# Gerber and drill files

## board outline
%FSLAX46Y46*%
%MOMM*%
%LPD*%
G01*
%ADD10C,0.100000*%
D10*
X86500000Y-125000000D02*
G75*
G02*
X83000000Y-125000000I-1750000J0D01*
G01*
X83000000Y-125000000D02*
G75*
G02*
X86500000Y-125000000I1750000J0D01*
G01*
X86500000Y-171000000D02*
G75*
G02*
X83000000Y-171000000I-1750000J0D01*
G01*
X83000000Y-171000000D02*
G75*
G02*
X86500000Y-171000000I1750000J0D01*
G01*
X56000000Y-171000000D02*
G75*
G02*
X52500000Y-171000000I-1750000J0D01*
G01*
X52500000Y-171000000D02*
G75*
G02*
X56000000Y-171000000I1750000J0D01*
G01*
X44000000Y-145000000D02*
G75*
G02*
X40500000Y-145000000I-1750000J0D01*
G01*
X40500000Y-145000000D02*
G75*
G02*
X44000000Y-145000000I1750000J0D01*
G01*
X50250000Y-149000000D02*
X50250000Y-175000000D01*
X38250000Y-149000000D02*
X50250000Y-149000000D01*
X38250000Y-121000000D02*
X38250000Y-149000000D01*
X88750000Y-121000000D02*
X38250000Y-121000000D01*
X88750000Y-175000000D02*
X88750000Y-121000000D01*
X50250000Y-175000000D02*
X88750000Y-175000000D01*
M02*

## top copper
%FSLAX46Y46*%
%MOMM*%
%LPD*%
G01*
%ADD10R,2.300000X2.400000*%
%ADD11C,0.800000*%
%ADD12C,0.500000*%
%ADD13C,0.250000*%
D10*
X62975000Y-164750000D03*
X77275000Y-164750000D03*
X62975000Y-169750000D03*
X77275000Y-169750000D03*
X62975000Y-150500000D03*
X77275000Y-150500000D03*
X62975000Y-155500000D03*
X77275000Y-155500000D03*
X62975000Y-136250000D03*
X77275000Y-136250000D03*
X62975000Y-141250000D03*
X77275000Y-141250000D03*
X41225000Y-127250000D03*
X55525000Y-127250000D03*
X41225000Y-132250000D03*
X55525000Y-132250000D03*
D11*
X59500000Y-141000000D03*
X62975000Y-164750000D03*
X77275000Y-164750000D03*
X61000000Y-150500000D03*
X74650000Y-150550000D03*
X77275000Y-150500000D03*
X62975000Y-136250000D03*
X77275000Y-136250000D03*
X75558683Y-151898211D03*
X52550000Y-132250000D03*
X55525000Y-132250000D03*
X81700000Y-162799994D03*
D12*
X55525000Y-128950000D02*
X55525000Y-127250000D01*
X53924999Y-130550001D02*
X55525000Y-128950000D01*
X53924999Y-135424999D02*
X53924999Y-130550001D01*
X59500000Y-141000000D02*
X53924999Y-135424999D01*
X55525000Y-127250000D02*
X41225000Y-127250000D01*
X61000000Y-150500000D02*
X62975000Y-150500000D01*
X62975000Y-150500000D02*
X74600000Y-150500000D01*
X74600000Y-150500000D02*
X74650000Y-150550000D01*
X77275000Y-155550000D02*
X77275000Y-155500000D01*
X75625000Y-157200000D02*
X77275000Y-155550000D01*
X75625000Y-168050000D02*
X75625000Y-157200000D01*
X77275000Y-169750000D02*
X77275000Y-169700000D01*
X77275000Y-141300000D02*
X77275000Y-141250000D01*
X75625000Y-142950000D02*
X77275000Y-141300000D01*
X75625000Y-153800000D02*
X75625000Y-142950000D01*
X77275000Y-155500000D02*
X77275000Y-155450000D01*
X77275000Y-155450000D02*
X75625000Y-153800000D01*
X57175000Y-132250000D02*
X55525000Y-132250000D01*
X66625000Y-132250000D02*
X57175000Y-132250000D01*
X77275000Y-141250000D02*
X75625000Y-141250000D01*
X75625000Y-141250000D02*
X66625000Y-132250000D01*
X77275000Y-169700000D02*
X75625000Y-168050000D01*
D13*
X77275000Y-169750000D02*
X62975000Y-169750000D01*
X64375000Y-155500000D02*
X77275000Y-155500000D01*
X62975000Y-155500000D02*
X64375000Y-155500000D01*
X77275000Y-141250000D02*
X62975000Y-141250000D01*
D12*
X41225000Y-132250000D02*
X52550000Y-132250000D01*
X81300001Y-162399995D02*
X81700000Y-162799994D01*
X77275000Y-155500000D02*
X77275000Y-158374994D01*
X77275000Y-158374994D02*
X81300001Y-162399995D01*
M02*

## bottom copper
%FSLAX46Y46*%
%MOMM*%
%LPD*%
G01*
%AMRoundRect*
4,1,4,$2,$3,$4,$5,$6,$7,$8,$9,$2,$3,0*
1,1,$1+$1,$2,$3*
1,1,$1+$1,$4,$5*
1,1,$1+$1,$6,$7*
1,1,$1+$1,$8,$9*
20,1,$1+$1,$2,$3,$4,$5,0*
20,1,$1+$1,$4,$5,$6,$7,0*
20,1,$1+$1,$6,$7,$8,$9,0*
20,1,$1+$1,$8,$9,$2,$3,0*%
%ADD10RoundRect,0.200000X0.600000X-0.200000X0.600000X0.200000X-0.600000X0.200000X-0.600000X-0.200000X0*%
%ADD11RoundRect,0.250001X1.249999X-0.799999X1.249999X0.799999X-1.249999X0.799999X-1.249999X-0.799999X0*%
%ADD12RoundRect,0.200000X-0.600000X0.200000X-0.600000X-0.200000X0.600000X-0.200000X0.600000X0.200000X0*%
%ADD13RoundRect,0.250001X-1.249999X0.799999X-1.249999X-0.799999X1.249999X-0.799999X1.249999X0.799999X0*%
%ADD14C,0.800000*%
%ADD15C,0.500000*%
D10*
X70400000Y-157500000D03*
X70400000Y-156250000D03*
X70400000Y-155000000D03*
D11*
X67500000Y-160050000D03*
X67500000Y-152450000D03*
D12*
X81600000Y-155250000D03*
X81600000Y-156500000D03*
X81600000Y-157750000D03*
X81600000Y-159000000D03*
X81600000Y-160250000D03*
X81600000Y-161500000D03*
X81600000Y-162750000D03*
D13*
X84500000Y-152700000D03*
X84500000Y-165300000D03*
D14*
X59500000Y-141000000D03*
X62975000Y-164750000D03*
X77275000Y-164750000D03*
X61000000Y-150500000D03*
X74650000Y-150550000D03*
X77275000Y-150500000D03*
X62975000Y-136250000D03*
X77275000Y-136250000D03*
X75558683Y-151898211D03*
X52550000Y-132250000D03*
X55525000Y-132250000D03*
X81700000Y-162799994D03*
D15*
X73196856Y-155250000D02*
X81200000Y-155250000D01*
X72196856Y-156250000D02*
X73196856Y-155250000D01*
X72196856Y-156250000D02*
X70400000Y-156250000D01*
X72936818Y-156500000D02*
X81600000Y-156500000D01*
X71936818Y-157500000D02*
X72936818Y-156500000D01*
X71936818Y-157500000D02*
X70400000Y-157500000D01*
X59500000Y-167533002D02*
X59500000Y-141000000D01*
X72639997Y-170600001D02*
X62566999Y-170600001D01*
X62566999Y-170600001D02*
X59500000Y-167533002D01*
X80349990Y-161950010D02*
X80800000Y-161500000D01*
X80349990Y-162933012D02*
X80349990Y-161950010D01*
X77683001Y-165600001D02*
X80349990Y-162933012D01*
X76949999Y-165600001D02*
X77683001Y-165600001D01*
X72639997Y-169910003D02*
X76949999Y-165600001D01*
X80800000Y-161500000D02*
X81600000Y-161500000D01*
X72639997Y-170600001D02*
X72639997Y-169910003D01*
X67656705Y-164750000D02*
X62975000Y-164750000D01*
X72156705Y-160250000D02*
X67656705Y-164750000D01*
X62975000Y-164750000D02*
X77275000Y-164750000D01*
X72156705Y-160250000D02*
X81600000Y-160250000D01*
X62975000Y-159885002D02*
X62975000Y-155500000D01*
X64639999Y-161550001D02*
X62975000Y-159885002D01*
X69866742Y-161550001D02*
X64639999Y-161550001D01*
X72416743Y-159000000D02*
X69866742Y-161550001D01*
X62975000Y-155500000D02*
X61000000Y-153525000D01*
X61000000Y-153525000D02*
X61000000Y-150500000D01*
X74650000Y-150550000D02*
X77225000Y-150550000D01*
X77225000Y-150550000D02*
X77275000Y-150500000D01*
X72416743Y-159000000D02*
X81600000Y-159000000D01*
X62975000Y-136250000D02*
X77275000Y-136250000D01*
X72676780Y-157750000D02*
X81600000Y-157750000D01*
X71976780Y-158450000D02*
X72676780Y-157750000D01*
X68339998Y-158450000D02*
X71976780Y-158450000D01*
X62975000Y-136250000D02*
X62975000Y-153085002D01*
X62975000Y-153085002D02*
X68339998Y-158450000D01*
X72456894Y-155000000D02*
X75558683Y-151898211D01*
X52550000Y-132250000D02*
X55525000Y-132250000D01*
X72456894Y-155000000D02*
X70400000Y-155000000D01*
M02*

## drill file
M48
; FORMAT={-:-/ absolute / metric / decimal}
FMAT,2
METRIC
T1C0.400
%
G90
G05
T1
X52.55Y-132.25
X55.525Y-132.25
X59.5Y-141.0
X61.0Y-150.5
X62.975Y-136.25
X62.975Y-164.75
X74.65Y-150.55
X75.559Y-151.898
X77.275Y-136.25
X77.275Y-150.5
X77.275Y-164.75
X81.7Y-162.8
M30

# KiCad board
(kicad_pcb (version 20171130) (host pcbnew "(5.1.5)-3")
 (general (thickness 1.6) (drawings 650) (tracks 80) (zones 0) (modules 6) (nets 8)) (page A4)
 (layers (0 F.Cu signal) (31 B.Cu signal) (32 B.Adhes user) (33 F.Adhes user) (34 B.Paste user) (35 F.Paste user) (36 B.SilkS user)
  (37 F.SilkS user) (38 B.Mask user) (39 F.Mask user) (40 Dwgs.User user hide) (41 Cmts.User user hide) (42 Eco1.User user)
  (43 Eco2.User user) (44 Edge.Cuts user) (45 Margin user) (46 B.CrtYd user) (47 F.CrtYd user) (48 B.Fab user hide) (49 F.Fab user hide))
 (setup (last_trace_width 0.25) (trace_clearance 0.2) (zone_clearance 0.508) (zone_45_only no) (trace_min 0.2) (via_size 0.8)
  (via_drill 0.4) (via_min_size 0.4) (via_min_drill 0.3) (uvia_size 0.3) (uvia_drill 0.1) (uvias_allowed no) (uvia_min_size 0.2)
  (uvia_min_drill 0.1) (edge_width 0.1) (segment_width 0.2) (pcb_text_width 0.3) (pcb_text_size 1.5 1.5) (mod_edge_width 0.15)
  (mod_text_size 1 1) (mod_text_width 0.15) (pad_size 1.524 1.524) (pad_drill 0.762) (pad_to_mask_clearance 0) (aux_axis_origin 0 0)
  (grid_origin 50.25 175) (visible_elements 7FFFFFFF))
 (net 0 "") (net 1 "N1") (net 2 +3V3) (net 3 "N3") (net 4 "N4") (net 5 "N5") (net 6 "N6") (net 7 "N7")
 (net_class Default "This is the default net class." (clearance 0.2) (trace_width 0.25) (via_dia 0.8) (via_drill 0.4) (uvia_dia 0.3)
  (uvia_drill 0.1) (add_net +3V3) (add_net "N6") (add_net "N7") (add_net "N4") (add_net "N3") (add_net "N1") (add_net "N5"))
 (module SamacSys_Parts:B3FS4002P (layer F.Cu) (at 71.25 167.25)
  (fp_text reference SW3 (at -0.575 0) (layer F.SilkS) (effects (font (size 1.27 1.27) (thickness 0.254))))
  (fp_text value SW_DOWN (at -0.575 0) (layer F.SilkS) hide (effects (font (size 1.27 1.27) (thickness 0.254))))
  (pad 2 smd rect (at -8.275 -2.5) (size 2.3 2.4) (layers F.Cu F.Paste F.Mask) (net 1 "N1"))
  (pad 2 smd rect (at 6.025 -2.5) (size 2.3 2.4) (layers F.Cu F.Paste F.Mask) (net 1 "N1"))
  (pad 1 smd rect (at -8.275 2.5) (size 2.3 2.4) (layers F.Cu F.Paste F.Mask) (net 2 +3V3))
  (pad 1 smd rect (at 6.025 2.5) (size 2.3 2.4) (layers F.Cu F.Paste F.Mask) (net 2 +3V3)))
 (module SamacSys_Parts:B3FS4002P (layer F.Cu) (at 71.25 153)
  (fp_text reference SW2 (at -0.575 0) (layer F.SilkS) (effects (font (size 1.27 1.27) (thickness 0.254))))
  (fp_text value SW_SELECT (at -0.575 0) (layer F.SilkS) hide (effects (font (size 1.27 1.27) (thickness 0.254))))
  (pad 2 smd rect (at -8.275 -2.5) (size 2.3 2.4) (layers F.Cu F.Paste F.Mask) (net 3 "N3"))
  (pad 2 smd rect (at 6.025 -2.5) (size 2.3 2.4) (layers F.Cu F.Paste F.Mask) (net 3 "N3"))
  (pad 1 smd rect (at -8.275 2.5) (size 2.3 2.4) (layers F.Cu F.Paste F.Mask) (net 2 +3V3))
  (pad 1 smd rect (at 6.025 2.5) (size 2.3 2.4) (layers F.Cu F.Paste F.Mask) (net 2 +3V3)))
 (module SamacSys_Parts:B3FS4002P (layer F.Cu) (at 71.25 138.75)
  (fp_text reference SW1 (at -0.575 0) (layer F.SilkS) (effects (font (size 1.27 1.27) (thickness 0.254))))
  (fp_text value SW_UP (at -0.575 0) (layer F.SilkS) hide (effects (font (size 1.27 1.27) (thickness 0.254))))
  (pad 2 smd rect (at -8.275 -2.5) (size 2.3 2.4) (layers F.Cu F.Paste F.Mask) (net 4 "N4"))
  (pad 2 smd rect (at 6.025 -2.5) (size 2.3 2.4) (layers F.Cu F.Paste F.Mask) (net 4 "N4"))
  (pad 1 smd rect (at -8.275 2.5) (size 2.3 2.4) (layers F.Cu F.Paste F.Mask) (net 2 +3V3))
  (pad 1 smd rect (at 6.025 2.5) (size 2.3 2.4) (layers F.Cu F.Paste F.Mask) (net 2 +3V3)))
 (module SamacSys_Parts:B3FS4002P (layer F.Cu) (at 49.5 129.75)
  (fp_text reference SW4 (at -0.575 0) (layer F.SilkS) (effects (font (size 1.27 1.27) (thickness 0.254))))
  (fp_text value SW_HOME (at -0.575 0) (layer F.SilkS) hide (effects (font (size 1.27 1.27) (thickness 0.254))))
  (pad 2 smd rect (at -8.275 -2.5) (size 2.3 2.4) (layers F.Cu F.Paste F.Mask) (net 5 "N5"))
  (pad 2 smd rect (at 6.025 -2.5) (size 2.3 2.4) (layers F.Cu F.Paste F.Mask) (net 5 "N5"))
  (pad 1 smd rect (at -8.275 2.5) (size 2.3 2.4) (layers F.Cu F.Paste F.Mask) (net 2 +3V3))
  (pad 1 smd rect (at 6.025 2.5) (size 2.3 2.4) (layers F.Cu F.Paste F.Mask) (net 2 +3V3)))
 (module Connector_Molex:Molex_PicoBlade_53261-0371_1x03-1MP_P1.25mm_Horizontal (layer B.Cu) (at 68 156.25 90)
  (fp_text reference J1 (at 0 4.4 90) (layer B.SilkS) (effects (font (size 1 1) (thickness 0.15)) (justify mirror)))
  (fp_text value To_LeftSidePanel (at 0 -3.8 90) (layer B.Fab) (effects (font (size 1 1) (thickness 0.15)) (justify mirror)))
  (pad 1 smd roundrect (at -1.25 2.4 90) (size 0.8 1.6) (layers B.Cu B.Paste B.Mask) (roundrect_rratio 0.25) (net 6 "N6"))
  (pad 2 smd roundrect (at 0 2.4 90) (size 0.8 1.6) (layers B.Cu B.Paste B.Mask) (roundrect_rratio 0.25) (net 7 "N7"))
  (pad 3 smd roundrect (at 1.25 2.4 90) (size 0.8 1.6) (layers B.Cu B.Paste B.Mask) (roundrect_rratio 0.25) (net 2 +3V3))
  (pad MP smd roundrect (at -3.8 -0.5 90) (size 2.1 3) (layers B.Cu B.Paste B.Mask) (roundrect_rratio 0.119048))
  (pad MP smd roundrect (at 3.8 -0.5 90) (size 2.1 3) (layers B.Cu B.Paste B.Mask) (roundrect_rratio 0.119048)))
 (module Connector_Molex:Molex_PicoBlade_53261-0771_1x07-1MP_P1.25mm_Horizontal (layer B.Cu) (at 84 159 270)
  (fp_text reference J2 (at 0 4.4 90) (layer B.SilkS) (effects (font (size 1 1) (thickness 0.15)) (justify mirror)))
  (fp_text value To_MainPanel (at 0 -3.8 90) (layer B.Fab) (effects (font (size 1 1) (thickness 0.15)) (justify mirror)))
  (pad 1 smd roundrect (at -3.75 2.4 270) (size 0.8 1.6) (layers B.Cu B.Paste B.Mask) (roundrect_rratio 0.25) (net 7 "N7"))
  (pad 2 smd roundrect (at -2.5 2.4 270) (size 0.8 1.6) (layers B.Cu B.Paste B.Mask) (roundrect_rratio 0.25) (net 6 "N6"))
  (pad 3 smd roundrect (at -1.25 2.4 270) (size 0.8 1.6) (layers B.Cu B.Paste B.Mask) (roundrect_rratio 0.25) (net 4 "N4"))
  (pad 4 smd roundrect (at 0 2.4 270) (size 0.8 1.6) (layers B.Cu B.Paste B.Mask) (roundrect_rratio 0.25) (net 3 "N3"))
  (pad 5 smd roundrect (at 1.25 2.4 270) (size 0.8 1.6) (layers B.Cu B.Paste B.Mask) (roundrect_rratio 0.25) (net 1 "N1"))
  (pad 6 smd roundrect (at 2.5 2.4 270) (size 0.8 1.6) (layers B.Cu B.Paste B.Mask) (roundrect_rratio 0.25) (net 5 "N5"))
  (pad 7 smd roundrect (at 3.75 2.4 270) (size 0.8 1.6) (layers B.Cu B.Paste B.Mask) (roundrect_rratio 0.25) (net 2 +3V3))
  (pad MP smd roundrect (at -6.3 -0.5 270) (size 2.1 3) (layers B.Cu B.Paste B.Mask) (roundrect_rratio 0.119048))
  (pad MP smd roundrect (at 6.3 -0.5 270) (size 2.1 3) (layers B.Cu B.Paste B.Mask) (roundrect_rratio 0.119048)))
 (gr_circle (center 84.75 125) (end 86.5 125) (layer Edge.Cuts) (width 0.1))
 (gr_circle (center 84.75 171) (end 86.5 171) (layer Edge.Cuts) (width 0.1))
 (gr_circle (center 54.25 171) (end 56 171) (layer Edge.Cuts) (width 0.1))
 (gr_circle (center 42.25 145) (end 44 145) (layer Edge.Cuts) (width 0.1))
 (gr_line (start 50.25 149) (end 50.25 175) (layer Edge.Cuts) (width 0.1))
 (gr_line (start 38.25 149) (end 50.25 149) (layer Edge.Cuts) (width 0.1))
 (gr_line (start 38.25 121) (end 38.25 149) (layer Edge.Cuts) (width 0.1))
 (gr_line (start 88.75 121) (end 38.25 121) (layer Edge.Cuts) (width 0.1))
 (gr_line (start 88.75 175) (end 88.75 121) (layer Edge.Cuts) (width 0.1))
 (gr_line (start 50.25 175) (end 88.75 175) (layer Edge.Cuts) (width 0.1))
 (segment (start 73.196856 155.25) (end 81.2 155.25) (width 0.5) (layer B.Cu) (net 7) (status 20))
 (segment (start 72.196856 156.25) (end 73.196856 155.25) (width 0.5) (layer B.Cu) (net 7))
 (segment (start 72.196856 156.25) (end 70.4 156.25) (width 0.5) (layer B.Cu) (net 7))
 (segment (start 72.936818 156.5) (end 81.6 156.5) (width 0.5) (layer B.Cu) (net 6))
 (segment (start 71.936818 157.5) (end 72.936818 156.5) (width 0.5) (layer B.Cu) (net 6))
 (segment (start 71.936818 157.5) (end 70.4 157.5) (width 0.5) (layer B.Cu) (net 6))
 (via (at 59.5 141) (size 0.8) (drill 0.4) (layers F.Cu B.Cu) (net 5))
 (segment (start 59.5 167.533002) (end 59.5 141) (width 0.5) (layer B.Cu) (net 5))
 (segment (start 72.639997 170.600001) (end 62.566999 170.600001) (width 0.5) (layer B.Cu) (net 5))
 (segment (start 62.566999 170.600001) (end 59.5 167.533002) (width 0.5) (layer B.Cu) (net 5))
 (segment (start 55.525 128.95) (end 55.525 127.25) (width 0.5) (layer F.Cu) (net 5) (status 20))
 (segment (start 53.924999 130.550001) (end 55.525 128.95) (width 0.5) (layer F.Cu) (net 5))
 (segment (start 53.924999 135.424999) (end 53.924999 130.550001) (width 0.5) (layer F.Cu) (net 5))
 (segment (start 59.5 141) (end 53.924999 135.424999) (width 0.5) (layer F.Cu) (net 5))
 (segment (start 55.525 127.25) (end 41.225 127.25) (width 0.5) (layer F.Cu) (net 5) (status 30))
 (segment (start 80.34999 161.95001) (end 80.8 161.5) (width 0.5) (layer B.Cu) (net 5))
 (segment (start 80.34999 162.933012) (end 80.34999 161.95001) (width 0.5) (layer B.Cu) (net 5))
 (segment (start 77.683001 165.600001) (end 80.34999 162.933012) (width 0.5) (layer B.Cu) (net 5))
 (segment (start 76.949999 165.600001) (end 77.683001 165.600001) (width 0.5) (layer B.Cu) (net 5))
 (segment (start 72.639997 169.910003) (end 76.949999 165.600001) (width 0.5) (layer B.Cu) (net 5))
 (segment (start 80.8 161.5) (end 81.6 161.5) (width 0.5) (layer B.Cu) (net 5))
 (segment (start 72.639997 170.600001) (end 72.639997 169.910003) (width 0.5) (layer B.Cu) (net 5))
 (via (at 62.975 164.75) (size 0.8) (drill 0.4) (layers F.Cu B.Cu) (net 1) (status 30))
 (segment (start 67.656705 164.75) (end 62.975 164.75) (width 0.5) (layer B.Cu) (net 1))
 (segment (start 72.156705 160.25) (end 67.656705 164.75) (width 0.5) (layer B.Cu) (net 1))
 (via (at 77.275 164.75) (size 0.8) (drill 0.4) (layers F.Cu B.Cu) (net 1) (status 30))
 (segment (start 62.975 164.75) (end 77.275 164.75) (width 0.5) (layer B.Cu) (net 1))
 (segment (start 72.156705 160.25) (end 81.6 160.25) (width 0.5) (layer B.Cu) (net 1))
 (segment (start 62.975 159.885002) (end 62.975 155.5) (width 0.5) (layer B.Cu) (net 3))
 (segment (start 64.639999 161.550001) (end 62.975 159.885002) (width 0.5) (layer B.Cu) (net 3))
 (segment (start 69.866742 161.550001) (end 64.639999 161.550001) (width 0.5) (layer B.Cu) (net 3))
 (segment (start 72.416743 159) (end 69.866742 161.550001) (width 0.5) (layer B.Cu) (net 3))
 (via (at 61 150.5) (size 0.8) (drill 0.4) (layers F.Cu B.Cu) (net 3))
 (segment (start 62.975 155.5) (end 61 153.525) (width 0.5) (layer B.Cu) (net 3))
 (segment (start 61 153.525) (end 61 150.5) (width 0.5) (layer B.Cu) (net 3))
 (segment (start 61 150.5) (end 62.975 150.5) (width 0.5) (layer F.Cu) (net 3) (status 20))
 (segment (start 62.975 150.5) (end 74.6 150.5) (width 0.5) (layer F.Cu) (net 3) (status 10))
 (via (at 74.65 150.55) (size 0.8) (drill 0.4) (layers F.Cu B.Cu) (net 3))
 (segment (start 74.6 150.5) (end 74.65 150.55) (width 0.5) (layer F.Cu) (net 3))
 (segment (start 74.65 150.55) (end 77.225 150.55) (width 0.5) (layer B.Cu) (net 3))
 (via (at 77.275 150.5) (size 0.8) (drill 0.4) (layers F.Cu B.Cu) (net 3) (status 30))
 (segment (start 77.225 150.55) (end 77.275 150.5) (width 0.5) (layer B.Cu) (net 3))
 (segment (start 72.416743 159) (end 81.6 159) (width 0.5) (layer B.Cu) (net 3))
 (via (at 62.975 136.25) (size 0.8) (drill 0.4) (layers F.Cu B.Cu) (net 4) (status 30))
 (via (at 77.275 136.25) (size 0.8) (drill 0.4) (layers F.Cu B.Cu) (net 4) (status 30))
 (segment (start 62.975 136.25) (end 77.275 136.25) (width 0.5) (layer B.Cu) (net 4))
 (segment (start 72.67678 157.75) (end 81.6 157.75) (width 0.5) (layer B.Cu) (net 4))
 (segment (start 71.97678 158.45) (end 72.67678 157.75) (width 0.5) (layer B.Cu) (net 4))
 (segment (start 68.339998 158.45) (end 71.97678 158.45) (width 0.5) (layer B.Cu) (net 4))
 (segment (start 62.975 136.25) (end 62.975 153.085002) (width 0.5) (layer B.Cu) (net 4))
 (segment (start 62.975 153.085002) (end 68.339998 158.45) (width 0.5) (layer B.Cu) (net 4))
 (segment (start 77.275 155.55) (end 77.275 155.5) (width 0.5) (layer F.Cu) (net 2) (status 30))
 (segment (start 75.625 157.2) (end 77.275 155.55) (width 0.5) (layer F.Cu) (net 2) (status 20))
 (segment (start 75.625 168.05) (end 75.625 157.2) (width 0.5) (layer F.Cu) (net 2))
 (segment (start 77.275 169.75) (end 77.275 169.7) (width 0.5) (layer F.Cu) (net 2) (status 30))
 (segment (start 77.275 141.3) (end 77.275 141.25) (width 0.5) (layer F.Cu) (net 2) (status 30))
 (segment (start 75.625 142.95) (end 77.275 141.3) (width 0.5) (layer F.Cu) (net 2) (status 20))
 (segment (start 75.625 153.8) (end 75.625 142.95) (width 0.5) (layer F.Cu) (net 2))
 (segment (start 77.275 155.5) (end 77.275 155.45) (width 0.5) (layer F.Cu) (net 2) (status 30))
 (segment (start 77.275 155.45) (end 75.625 153.8) (width 0.5) (layer F.Cu) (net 2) (status 10))
 (segment (start 57.175 132.25) (end 55.525 132.25) (width 0.5) (layer F.Cu) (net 2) (status 20))
 (segment (start 66.625 132.25) (end 57.175 132.25) (width 0.5) (layer F.Cu) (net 2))
 (segment (start 77.275 141.25) (end 75.625 141.25) (width 0.5) (layer F.Cu) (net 2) (status 10))
 (segment (start 75.625 141.25) (end 66.625 132.25) (width 0.5) (layer F.Cu) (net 2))
 (via (at 75.558683 151.898211) (size 0.8) (drill 0.4) (layers F.Cu B.Cu) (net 2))
 (segment (start 72.456894 155) (end 75.558683 151.898211) (width 0.5) (layer B.Cu) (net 2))
 (segment (start 77.275 169.7) (end 75.625 168.05) (width 0.5) (layer F.Cu) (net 2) (status 10))
 (segment (start 77.275 169.75) (end 62.975 169.75) (width 0.25) (layer F.Cu) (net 2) (status 30))
 (segment (start 64.375 155.5) (end 77.275 155.5) (width 0.25) (layer F.Cu) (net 2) (status 20))
 (segment (start 62.975 155.5) (end 64.375 155.5) (width 0.25) (layer F.Cu) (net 2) (status 10))
 (segment (start 77.275 141.25) (end 62.975 141.25) (width 0.25) (layer F.Cu) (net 2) (status 30))
 (via (at 52.55 132.25) (size 0.8) (drill 0.4) (layers F.Cu B.Cu) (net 2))
 (segment (start 41.225 132.25) (end 52.55 132.25) (width 0.5) (layer F.Cu) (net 2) (status 10))
 (via (at 55.525 132.25) (size 0.8) (drill 0.4) (layers F.Cu B.Cu) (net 2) (status 30))
 (segment (start 52.55 132.25) (end 55.525 132.25) (width 0.5) (layer B.Cu) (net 2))
 (via (at 81.7 162.799994) (size 0.8) (drill 0.4) (layers F.Cu B.Cu) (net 2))
 (segment (start 81.300001 162.399995) (end 81.7 162.799994) (width 0.5) (layer F.Cu) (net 2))
 (segment (start 77.275 155.5) (end 77.275 158.374994) (width 0.5) (layer F.Cu) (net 2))
 (segment (start 77.275 158.374994) (end 81.300001 162.399995) (width 0.5) (layer F.Cu) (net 2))
 (segment (start 72.456894 155) (end 70.4 155) (width 0.5) (layer B.Cu) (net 2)))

